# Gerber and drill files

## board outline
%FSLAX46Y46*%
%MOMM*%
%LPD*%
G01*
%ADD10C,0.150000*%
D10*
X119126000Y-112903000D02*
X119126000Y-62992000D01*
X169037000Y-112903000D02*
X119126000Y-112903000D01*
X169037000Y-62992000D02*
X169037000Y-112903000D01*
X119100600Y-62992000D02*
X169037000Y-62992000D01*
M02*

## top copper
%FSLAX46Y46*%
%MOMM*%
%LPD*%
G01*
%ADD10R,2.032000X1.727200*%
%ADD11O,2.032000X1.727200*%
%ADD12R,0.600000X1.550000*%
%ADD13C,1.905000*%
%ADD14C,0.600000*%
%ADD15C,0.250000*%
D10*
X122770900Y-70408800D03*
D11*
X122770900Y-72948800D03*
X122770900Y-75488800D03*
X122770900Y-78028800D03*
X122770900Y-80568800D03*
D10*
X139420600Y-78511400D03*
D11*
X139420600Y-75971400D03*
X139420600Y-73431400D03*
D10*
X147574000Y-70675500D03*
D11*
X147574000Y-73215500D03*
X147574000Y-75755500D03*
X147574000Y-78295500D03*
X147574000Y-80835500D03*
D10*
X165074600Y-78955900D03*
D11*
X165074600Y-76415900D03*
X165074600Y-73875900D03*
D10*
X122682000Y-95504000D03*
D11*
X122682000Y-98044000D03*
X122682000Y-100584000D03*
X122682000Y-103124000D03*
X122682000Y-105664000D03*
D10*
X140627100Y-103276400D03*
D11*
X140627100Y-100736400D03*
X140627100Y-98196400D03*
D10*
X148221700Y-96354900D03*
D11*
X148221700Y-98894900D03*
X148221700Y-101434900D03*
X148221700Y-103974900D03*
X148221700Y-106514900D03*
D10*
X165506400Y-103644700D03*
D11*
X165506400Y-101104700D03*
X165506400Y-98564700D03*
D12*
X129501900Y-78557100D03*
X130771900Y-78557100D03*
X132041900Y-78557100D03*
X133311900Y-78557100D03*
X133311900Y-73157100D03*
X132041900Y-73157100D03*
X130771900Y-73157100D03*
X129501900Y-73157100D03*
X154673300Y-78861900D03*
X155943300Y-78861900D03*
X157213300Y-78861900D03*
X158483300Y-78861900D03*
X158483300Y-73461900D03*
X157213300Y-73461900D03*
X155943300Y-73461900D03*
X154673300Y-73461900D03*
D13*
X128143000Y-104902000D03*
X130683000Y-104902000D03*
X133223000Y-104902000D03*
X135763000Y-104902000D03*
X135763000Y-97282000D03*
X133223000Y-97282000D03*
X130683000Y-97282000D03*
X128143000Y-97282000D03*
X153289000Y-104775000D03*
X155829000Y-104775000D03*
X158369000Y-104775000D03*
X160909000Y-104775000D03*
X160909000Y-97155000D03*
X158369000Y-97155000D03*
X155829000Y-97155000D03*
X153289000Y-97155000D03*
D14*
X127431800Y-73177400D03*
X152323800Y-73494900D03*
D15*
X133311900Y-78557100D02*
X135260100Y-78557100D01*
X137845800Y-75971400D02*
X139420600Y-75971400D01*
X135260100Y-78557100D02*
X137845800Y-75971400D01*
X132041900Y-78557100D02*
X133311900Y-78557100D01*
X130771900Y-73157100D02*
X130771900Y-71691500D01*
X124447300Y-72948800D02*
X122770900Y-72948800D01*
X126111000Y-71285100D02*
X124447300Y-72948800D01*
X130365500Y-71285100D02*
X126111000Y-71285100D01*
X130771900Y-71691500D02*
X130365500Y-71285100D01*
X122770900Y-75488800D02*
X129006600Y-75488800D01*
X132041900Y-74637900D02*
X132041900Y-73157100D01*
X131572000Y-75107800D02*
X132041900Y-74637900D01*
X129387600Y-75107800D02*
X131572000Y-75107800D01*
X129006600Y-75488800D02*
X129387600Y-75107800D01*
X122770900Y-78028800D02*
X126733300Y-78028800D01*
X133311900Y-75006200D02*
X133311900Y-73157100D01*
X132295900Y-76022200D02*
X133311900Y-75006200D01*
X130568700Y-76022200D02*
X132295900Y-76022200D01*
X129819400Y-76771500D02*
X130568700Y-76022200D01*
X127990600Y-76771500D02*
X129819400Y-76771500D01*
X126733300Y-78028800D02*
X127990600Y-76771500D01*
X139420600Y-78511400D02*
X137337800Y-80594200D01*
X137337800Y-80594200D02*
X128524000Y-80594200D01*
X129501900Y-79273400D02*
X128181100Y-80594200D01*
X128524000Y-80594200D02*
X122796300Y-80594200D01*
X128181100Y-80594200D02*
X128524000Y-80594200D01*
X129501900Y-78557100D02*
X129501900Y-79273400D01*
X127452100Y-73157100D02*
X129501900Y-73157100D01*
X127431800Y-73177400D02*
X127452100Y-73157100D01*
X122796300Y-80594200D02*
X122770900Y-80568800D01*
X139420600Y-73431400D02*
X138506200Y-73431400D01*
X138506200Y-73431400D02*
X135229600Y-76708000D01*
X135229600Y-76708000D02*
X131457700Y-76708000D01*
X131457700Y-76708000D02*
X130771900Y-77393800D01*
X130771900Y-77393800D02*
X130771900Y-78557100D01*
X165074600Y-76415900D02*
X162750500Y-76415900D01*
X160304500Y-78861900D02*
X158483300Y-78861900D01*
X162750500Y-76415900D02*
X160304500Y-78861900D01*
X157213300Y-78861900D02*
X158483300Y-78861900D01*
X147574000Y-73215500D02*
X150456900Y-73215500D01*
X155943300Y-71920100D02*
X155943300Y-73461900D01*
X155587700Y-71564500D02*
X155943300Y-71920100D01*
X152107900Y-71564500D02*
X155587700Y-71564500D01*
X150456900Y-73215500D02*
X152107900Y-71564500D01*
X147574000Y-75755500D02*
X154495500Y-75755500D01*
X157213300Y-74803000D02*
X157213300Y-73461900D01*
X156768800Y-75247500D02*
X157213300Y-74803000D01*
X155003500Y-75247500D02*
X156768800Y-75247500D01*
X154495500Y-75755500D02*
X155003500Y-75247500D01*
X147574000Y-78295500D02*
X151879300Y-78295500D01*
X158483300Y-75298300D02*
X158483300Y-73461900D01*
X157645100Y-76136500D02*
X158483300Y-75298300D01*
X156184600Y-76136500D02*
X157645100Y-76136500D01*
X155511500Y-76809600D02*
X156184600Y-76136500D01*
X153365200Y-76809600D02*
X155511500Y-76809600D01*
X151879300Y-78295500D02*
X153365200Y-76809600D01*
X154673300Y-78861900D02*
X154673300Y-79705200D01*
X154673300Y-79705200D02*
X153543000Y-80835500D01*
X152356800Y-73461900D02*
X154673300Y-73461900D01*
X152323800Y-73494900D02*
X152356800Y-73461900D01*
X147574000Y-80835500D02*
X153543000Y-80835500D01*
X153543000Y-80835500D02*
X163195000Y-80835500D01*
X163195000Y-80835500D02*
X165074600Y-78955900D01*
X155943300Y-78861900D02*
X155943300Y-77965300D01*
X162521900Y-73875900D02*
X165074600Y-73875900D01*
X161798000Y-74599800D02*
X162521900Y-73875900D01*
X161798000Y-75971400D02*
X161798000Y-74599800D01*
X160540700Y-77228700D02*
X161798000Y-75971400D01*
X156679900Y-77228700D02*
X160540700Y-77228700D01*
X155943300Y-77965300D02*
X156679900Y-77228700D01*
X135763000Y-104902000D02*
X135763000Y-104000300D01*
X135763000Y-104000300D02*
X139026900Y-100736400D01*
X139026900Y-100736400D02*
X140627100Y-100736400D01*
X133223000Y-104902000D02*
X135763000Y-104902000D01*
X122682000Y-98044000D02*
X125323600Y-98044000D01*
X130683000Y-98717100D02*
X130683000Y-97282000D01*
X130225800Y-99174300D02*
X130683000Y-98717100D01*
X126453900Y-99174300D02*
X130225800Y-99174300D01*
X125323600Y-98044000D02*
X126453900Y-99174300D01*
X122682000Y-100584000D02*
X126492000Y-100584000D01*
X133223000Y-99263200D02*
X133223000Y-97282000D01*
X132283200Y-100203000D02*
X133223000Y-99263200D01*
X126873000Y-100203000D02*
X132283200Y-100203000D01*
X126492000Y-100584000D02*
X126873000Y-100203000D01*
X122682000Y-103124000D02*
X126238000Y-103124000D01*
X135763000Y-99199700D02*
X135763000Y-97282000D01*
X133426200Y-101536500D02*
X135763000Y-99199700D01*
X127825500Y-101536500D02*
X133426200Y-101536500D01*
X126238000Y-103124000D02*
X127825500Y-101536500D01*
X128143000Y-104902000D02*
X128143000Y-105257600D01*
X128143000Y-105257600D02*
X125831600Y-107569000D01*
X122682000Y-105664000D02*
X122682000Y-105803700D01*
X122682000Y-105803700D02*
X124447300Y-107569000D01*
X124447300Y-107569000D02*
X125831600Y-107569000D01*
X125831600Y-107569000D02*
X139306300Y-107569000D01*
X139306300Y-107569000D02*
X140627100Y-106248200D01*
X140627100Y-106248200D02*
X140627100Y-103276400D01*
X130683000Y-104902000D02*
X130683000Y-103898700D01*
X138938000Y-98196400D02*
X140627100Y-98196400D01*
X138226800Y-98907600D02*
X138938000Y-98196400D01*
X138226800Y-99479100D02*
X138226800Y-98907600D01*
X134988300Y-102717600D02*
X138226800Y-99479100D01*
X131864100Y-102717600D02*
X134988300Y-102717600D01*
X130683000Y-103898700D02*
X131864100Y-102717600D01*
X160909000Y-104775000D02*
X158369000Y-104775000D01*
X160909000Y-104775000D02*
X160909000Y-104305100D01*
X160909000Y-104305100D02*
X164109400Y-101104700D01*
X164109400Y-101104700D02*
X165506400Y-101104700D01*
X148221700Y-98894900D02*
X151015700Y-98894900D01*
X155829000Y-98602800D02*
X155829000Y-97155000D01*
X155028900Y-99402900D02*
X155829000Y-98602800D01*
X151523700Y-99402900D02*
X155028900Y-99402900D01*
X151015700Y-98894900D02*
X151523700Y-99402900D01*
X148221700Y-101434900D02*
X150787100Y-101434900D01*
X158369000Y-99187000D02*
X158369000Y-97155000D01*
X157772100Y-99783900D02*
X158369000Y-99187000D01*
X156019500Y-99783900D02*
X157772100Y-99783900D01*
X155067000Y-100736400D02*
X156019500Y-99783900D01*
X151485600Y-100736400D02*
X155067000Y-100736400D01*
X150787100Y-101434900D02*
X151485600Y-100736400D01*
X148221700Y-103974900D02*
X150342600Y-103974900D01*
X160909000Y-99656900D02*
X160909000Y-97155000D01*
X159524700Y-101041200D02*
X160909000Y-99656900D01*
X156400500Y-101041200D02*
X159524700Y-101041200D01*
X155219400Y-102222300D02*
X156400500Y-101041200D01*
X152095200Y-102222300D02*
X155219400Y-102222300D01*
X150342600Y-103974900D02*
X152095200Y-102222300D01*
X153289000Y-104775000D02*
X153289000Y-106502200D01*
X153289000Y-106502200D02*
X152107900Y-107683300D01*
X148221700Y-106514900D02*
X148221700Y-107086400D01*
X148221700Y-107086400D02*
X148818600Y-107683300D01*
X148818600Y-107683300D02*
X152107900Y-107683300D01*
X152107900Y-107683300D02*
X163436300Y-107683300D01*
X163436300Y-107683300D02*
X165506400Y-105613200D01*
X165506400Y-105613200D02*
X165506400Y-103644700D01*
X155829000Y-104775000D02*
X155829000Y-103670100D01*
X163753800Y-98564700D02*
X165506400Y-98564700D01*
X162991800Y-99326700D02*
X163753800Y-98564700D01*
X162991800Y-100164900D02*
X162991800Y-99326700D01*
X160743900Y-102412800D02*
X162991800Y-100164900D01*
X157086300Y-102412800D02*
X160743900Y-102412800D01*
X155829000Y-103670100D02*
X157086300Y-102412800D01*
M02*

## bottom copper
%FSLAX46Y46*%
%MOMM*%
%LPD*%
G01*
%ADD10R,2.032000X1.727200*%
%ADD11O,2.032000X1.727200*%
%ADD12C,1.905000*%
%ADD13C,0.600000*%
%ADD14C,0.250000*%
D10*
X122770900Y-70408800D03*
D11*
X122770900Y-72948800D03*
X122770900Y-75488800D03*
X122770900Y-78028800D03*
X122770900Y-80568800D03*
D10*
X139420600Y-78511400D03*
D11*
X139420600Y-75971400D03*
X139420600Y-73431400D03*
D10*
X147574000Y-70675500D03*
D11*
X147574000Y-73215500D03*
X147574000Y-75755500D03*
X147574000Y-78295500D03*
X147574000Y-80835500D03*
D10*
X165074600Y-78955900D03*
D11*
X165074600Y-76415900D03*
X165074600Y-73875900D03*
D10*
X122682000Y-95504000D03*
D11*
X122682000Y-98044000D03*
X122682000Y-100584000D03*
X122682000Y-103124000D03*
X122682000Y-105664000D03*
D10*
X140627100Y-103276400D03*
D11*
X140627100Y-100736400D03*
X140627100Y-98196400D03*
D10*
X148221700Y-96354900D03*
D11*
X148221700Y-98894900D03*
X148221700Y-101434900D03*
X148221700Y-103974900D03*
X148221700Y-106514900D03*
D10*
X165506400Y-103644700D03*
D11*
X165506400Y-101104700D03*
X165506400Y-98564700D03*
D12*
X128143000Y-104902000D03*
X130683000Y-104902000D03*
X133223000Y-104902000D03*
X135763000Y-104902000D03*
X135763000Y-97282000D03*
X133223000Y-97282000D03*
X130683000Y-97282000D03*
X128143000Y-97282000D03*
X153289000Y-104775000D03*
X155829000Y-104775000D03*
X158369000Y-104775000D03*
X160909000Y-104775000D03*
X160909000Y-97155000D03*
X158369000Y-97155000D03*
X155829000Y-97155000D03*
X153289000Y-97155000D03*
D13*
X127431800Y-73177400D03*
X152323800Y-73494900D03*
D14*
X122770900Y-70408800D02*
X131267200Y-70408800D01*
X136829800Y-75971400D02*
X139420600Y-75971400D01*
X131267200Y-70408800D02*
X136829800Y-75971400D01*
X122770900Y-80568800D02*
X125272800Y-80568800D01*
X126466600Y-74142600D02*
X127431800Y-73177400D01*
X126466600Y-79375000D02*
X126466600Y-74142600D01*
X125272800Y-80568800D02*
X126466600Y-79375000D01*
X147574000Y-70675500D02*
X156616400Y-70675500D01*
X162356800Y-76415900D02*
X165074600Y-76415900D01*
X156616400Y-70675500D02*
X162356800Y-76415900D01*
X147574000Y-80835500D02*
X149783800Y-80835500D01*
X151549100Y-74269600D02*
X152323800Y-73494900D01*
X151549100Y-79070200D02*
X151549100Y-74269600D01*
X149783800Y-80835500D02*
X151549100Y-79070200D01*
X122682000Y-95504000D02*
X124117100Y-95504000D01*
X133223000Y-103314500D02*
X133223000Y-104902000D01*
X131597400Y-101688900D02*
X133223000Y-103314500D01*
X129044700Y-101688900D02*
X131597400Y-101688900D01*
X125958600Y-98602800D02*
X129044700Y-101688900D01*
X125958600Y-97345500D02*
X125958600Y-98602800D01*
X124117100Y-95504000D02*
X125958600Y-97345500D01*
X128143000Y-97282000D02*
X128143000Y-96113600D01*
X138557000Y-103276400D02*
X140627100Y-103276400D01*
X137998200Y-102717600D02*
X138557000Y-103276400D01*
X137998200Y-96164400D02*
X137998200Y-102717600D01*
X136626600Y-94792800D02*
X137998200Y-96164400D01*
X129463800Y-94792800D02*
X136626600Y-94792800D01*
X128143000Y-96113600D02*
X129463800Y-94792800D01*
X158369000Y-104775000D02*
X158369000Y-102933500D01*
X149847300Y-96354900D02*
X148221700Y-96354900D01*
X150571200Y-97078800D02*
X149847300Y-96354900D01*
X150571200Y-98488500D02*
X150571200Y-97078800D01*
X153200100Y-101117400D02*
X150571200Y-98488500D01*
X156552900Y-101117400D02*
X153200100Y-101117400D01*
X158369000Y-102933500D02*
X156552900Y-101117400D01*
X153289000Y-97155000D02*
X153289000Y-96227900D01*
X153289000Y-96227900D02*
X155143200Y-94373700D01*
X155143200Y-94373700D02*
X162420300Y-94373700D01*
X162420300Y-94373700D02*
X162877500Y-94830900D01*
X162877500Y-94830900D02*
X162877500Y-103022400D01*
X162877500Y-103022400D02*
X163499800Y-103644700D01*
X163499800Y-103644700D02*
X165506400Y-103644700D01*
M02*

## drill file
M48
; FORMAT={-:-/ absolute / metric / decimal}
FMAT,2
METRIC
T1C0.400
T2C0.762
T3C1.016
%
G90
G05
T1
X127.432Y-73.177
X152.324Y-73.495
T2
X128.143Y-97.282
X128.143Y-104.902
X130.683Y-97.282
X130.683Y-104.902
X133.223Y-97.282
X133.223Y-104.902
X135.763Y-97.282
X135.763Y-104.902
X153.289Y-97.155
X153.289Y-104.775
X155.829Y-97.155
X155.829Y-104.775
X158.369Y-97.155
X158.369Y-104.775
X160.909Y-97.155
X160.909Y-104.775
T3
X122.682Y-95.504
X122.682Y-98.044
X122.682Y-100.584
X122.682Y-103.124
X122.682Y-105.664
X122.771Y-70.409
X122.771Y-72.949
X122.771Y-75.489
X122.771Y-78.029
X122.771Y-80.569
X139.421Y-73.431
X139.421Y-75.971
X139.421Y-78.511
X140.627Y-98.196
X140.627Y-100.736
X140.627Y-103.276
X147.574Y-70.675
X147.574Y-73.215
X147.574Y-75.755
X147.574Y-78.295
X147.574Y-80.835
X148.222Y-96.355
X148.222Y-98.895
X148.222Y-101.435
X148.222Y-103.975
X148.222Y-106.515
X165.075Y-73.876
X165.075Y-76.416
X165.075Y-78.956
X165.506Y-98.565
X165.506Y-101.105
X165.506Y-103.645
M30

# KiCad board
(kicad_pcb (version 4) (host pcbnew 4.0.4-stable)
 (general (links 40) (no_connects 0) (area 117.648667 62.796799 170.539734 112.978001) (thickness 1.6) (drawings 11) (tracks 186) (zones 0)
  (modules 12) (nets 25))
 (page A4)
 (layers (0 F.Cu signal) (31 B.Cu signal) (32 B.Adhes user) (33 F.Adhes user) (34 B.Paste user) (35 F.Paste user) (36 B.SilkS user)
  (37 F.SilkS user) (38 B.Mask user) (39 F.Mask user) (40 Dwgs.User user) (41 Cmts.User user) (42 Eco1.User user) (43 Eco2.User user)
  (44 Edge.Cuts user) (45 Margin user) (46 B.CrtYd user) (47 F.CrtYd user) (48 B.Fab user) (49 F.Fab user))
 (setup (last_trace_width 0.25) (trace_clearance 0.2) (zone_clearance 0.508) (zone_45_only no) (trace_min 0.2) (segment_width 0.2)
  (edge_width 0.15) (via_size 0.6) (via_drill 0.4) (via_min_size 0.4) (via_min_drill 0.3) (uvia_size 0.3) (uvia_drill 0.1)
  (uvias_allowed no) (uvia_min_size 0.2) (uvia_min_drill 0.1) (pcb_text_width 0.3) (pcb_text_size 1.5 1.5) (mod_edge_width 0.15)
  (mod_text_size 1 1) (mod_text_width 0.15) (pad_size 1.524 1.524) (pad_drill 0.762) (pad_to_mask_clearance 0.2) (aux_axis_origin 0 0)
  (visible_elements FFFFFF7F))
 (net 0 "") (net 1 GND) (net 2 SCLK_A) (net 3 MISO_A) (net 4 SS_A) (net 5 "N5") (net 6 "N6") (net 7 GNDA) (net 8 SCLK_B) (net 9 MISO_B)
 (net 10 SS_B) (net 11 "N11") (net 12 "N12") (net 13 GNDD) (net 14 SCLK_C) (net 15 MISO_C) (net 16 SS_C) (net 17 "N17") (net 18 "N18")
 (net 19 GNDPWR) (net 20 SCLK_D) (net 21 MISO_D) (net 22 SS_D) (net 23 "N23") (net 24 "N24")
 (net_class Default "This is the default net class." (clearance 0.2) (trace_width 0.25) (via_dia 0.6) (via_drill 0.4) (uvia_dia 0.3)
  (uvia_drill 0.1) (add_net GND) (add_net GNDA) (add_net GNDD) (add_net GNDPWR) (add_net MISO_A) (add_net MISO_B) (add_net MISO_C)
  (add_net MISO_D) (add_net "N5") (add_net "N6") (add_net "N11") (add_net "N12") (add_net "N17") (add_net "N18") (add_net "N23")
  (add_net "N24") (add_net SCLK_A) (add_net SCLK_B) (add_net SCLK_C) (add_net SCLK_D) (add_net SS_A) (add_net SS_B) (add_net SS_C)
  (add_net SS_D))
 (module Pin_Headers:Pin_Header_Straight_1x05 (layer F.Cu) (at 122.7709 70.4088)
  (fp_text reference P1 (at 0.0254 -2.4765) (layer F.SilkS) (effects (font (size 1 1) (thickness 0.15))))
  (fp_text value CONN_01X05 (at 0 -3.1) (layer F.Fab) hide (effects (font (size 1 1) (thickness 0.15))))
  (pad 1 thru_hole rect (at 0 0) (size 2.032 1.7272) (drill 1.016) (layers *.Cu *.Mask) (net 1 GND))
  (pad 2 thru_hole oval (at 0 2.54) (size 2.032 1.7272) (drill 1.016) (layers *.Cu *.Mask) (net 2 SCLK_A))
  (pad 3 thru_hole oval (at 0 5.08) (size 2.032 1.7272) (drill 1.016) (layers *.Cu *.Mask) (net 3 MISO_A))
  (pad 4 thru_hole oval (at 0 7.62) (size 2.032 1.7272) (drill 1.016) (layers *.Cu *.Mask) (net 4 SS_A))
  (pad 5 thru_hole oval (at 0 10.16) (size 2.032 1.7272) (drill 1.016) (layers *.Cu *.Mask) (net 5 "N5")))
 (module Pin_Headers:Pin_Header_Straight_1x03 (layer F.Cu) (at 139.4206 78.5114 180)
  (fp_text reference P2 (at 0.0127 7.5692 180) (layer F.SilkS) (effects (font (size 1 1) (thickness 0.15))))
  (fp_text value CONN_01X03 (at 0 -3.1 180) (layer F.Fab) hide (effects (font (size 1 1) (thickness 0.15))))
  (pad 1 thru_hole rect (at 0 0 180) (size 2.032 1.7272) (drill 1.016) (layers *.Cu *.Mask) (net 5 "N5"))
  (pad 2 thru_hole oval (at 0 2.54 180) (size 2.032 1.7272) (drill 1.016) (layers *.Cu *.Mask) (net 1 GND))
  (pad 3 thru_hole oval (at 0 5.08 180) (size 2.032 1.7272) (drill 1.016) (layers *.Cu *.Mask) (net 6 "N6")))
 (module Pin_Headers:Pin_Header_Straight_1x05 (layer F.Cu) (at 147.574 70.6755)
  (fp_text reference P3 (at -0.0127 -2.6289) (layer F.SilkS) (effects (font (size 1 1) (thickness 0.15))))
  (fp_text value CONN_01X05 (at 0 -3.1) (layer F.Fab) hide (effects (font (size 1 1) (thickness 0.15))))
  (pad 1 thru_hole rect (at 0 0) (size 2.032 1.7272) (drill 1.016) (layers *.Cu *.Mask) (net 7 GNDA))
  (pad 2 thru_hole oval (at 0 2.54) (size 2.032 1.7272) (drill 1.016) (layers *.Cu *.Mask) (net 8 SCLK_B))
  (pad 3 thru_hole oval (at 0 5.08) (size 2.032 1.7272) (drill 1.016) (layers *.Cu *.Mask) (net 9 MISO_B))
  (pad 4 thru_hole oval (at 0 7.62) (size 2.032 1.7272) (drill 1.016) (layers *.Cu *.Mask) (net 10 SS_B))
  (pad 5 thru_hole oval (at 0 10.16) (size 2.032 1.7272) (drill 1.016) (layers *.Cu *.Mask) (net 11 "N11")))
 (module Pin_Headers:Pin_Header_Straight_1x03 (layer F.Cu) (at 165.0746 78.9559 180)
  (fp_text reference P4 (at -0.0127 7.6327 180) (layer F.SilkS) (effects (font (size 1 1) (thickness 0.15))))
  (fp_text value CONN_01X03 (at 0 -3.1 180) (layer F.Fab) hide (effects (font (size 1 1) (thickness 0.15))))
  (pad 1 thru_hole rect (at 0 0 180) (size 2.032 1.7272) (drill 1.016) (layers *.Cu *.Mask) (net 11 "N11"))
  (pad 2 thru_hole oval (at 0 2.54 180) (size 2.032 1.7272) (drill 1.016) (layers *.Cu *.Mask) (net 7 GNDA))
  (pad 3 thru_hole oval (at 0 5.08 180) (size 2.032 1.7272) (drill 1.016) (layers *.Cu *.Mask) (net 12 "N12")))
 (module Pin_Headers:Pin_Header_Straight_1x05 (layer F.Cu) (at 122.682 95.504)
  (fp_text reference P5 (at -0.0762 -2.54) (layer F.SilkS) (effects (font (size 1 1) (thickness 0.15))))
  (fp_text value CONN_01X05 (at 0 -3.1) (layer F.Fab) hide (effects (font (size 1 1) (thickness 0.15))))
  (pad 1 thru_hole rect (at 0 0) (size 2.032 1.7272) (drill 1.016) (layers *.Cu *.Mask) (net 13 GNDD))
  (pad 2 thru_hole oval (at 0 2.54) (size 2.032 1.7272) (drill 1.016) (layers *.Cu *.Mask) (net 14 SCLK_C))
  (pad 3 thru_hole oval (at 0 5.08) (size 2.032 1.7272) (drill 1.016) (layers *.Cu *.Mask) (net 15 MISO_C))
  (pad 4 thru_hole oval (at 0 7.62) (size 2.032 1.7272) (drill 1.016) (layers *.Cu *.Mask) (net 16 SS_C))
  (pad 5 thru_hole oval (at 0 10.16) (size 2.032 1.7272) (drill 1.016) (layers *.Cu *.Mask) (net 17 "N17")))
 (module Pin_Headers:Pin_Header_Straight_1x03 (layer F.Cu) (at 140.6271 103.2764 180)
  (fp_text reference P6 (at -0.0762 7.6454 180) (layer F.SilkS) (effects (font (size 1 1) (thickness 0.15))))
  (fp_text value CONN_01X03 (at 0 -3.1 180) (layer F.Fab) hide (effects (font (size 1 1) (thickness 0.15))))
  (pad 1 thru_hole rect (at 0 0 180) (size 2.032 1.7272) (drill 1.016) (layers *.Cu *.Mask) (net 17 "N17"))
  (pad 2 thru_hole oval (at 0 2.54 180) (size 2.032 1.7272) (drill 1.016) (layers *.Cu *.Mask) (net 13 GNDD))
  (pad 3 thru_hole oval (at 0 5.08 180) (size 2.032 1.7272) (drill 1.016) (layers *.Cu *.Mask) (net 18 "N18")))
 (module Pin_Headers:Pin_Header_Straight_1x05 (layer F.Cu) (at 148.2217 96.3549)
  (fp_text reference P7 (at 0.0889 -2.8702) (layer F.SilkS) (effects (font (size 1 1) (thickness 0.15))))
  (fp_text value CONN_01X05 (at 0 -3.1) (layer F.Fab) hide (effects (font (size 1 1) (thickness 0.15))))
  (pad 1 thru_hole rect (at 0 0) (size 2.032 1.7272) (drill 1.016) (layers *.Cu *.Mask) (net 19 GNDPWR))
  (pad 2 thru_hole oval (at 0 2.54) (size 2.032 1.7272) (drill 1.016) (layers *.Cu *.Mask) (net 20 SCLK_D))
  (pad 3 thru_hole oval (at 0 5.08) (size 2.032 1.7272) (drill 1.016) (layers *.Cu *.Mask) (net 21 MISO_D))
  (pad 4 thru_hole oval (at 0 7.62) (size 2.032 1.7272) (drill 1.016) (layers *.Cu *.Mask) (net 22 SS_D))
  (pad 5 thru_hole oval (at 0 10.16) (size 2.032 1.7272) (drill 1.016) (layers *.Cu *.Mask) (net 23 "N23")))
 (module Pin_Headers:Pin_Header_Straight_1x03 (layer F.Cu) (at 165.5064 103.6447 180)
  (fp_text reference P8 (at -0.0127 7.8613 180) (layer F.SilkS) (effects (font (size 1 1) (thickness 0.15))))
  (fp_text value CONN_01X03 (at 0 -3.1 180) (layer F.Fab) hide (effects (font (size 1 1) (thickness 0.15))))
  (pad 1 thru_hole rect (at 0 0 180) (size 2.032 1.7272) (drill 1.016) (layers *.Cu *.Mask) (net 23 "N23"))
  (pad 2 thru_hole oval (at 0 2.54 180) (size 2.032 1.7272) (drill 1.016) (layers *.Cu *.Mask) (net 19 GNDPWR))
  (pad 3 thru_hole oval (at 0 5.08 180) (size 2.032 1.7272) (drill 1.016) (layers *.Cu *.Mask) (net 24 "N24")))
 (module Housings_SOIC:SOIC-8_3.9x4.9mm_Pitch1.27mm (layer F.Cu) (at 131.4069 75.8571 90)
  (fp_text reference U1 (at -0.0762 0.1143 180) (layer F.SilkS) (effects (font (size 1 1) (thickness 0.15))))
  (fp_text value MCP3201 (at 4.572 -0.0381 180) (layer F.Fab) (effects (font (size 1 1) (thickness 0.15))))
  (pad 1 smd rect (at -2.7 -1.905 90) (size 1.55 0.6) (layers F.Cu F.Paste F.Mask) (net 5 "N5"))
  (pad 2 smd rect (at -2.7 -0.635 90) (size 1.55 0.6) (layers F.Cu F.Paste F.Mask) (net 6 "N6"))
  (pad 3 smd rect (at -2.7 0.635 90) (size 1.55 0.6) (layers F.Cu F.Paste F.Mask) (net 1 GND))
  (pad 4 smd rect (at -2.7 1.905 90) (size 1.55 0.6) (layers F.Cu F.Paste F.Mask) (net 1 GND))
  (pad 5 smd rect (at 2.7 1.905 90) (size 1.55 0.6) (layers F.Cu F.Paste F.Mask) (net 4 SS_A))
  (pad 6 smd rect (at 2.7 0.635 90) (size 1.55 0.6) (layers F.Cu F.Paste F.Mask) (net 3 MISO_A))
  (pad 7 smd rect (at 2.7 -0.635 90) (size 1.55 0.6) (layers F.Cu F.Paste F.Mask) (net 2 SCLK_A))
  (pad 8 smd rect (at 2.7 -1.905 90) (size 1.55 0.6) (layers F.Cu F.Paste F.Mask) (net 5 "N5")))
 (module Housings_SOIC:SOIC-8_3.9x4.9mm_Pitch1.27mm (layer F.Cu) (at 156.5783 76.1619 90)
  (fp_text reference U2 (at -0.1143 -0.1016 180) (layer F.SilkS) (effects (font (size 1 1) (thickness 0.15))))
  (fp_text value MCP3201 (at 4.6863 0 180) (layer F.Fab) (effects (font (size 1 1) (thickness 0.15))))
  (pad 1 smd rect (at -2.7 -1.905 90) (size 1.55 0.6) (layers F.Cu F.Paste F.Mask) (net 11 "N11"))
  (pad 2 smd rect (at -2.7 -0.635 90) (size 1.55 0.6) (layers F.Cu F.Paste F.Mask) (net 12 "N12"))
  (pad 3 smd rect (at -2.7 0.635 90) (size 1.55 0.6) (layers F.Cu F.Paste F.Mask) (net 7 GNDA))
  (pad 4 smd rect (at -2.7 1.905 90) (size 1.55 0.6) (layers F.Cu F.Paste F.Mask) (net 7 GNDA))
  (pad 5 smd rect (at 2.7 1.905 90) (size 1.55 0.6) (layers F.Cu F.Paste F.Mask) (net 10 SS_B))
  (pad 6 smd rect (at 2.7 0.635 90) (size 1.55 0.6) (layers F.Cu F.Paste F.Mask) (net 9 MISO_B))
  (pad 7 smd rect (at 2.7 -0.635 90) (size 1.55 0.6) (layers F.Cu F.Paste F.Mask) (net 8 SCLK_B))
  (pad 8 smd rect (at 2.7 -1.905 90) (size 1.55 0.6) (layers F.Cu F.Paste F.Mask) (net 11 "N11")))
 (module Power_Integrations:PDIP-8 (layer F.Cu) (at 131.953 101.092)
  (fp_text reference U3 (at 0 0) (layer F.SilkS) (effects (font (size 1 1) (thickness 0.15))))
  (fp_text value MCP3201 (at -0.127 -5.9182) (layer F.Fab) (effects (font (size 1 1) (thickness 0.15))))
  (pad 1 thru_hole circle (at -3.81 3.81) (size 1.905 1.905) (drill 0.762) (layers *.Cu *.Mask) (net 17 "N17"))
  (pad 2 thru_hole circle (at -1.27 3.81) (size 1.905 1.905) (drill 0.762) (layers *.Cu *.Mask) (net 18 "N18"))
  (pad 3 thru_hole circle (at 1.27 3.81) (size 1.905 1.905) (drill 0.762) (layers *.Cu *.Mask) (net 13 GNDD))
  (pad 4 thru_hole circle (at 3.81 3.81) (size 1.905 1.905) (drill 0.762) (layers *.Cu *.Mask) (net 13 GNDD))
  (pad 5 thru_hole circle (at 3.81 -3.81) (size 1.905 1.905) (drill 0.762) (layers *.Cu *.Mask) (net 16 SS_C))
  (pad 6 thru_hole circle (at 1.27 -3.81) (size 1.905 1.905) (drill 0.762) (layers *.Cu *.Mask) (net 15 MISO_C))
  (pad 7 thru_hole circle (at -1.27 -3.81) (size 1.905 1.905) (drill 0.762) (layers *.Cu *.Mask) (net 14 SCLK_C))
  (pad 8 thru_hole circle (at -3.81 -3.81) (size 1.905 1.905) (drill 0.762) (layers *.Cu *.Mask) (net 17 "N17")))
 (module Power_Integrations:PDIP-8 (layer F.Cu) (at 157.099 100.965)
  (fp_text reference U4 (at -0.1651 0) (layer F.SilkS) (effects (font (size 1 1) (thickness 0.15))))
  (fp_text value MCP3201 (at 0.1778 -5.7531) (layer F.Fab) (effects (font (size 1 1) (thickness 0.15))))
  (pad 1 thru_hole circle (at -3.81 3.81) (size 1.905 1.905) (drill 0.762) (layers *.Cu *.Mask) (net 23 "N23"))
  (pad 2 thru_hole circle (at -1.27 3.81) (size 1.905 1.905) (drill 0.762) (layers *.Cu *.Mask) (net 24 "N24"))
  (pad 3 thru_hole circle (at 1.27 3.81) (size 1.905 1.905) (drill 0.762) (layers *.Cu *.Mask) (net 19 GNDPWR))
  (pad 4 thru_hole circle (at 3.81 3.81) (size 1.905 1.905) (drill 0.762) (layers *.Cu *.Mask) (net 19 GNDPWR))
  (pad 5 thru_hole circle (at 3.81 -3.81) (size 1.905 1.905) (drill 0.762) (layers *.Cu *.Mask) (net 22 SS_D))
  (pad 6 thru_hole circle (at 1.27 -3.81) (size 1.905 1.905) (drill 0.762) (layers *.Cu *.Mask) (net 21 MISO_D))
  (pad 7 thru_hole circle (at -1.27 -3.81) (size 1.905 1.905) (drill 0.762) (layers *.Cu *.Mask) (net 20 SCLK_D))
  (pad 8 thru_hole circle (at -3.81 -3.81) (size 1.905 1.905) (drill 0.762) (layers *.Cu *.Mask) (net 23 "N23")))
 (gr_line (start 119.126 112.903) (end 119.126 62.992) (angle 90) (layer Edge.Cuts) (width 0.15))
 (gr_line (start 169.037 112.903) (end 119.126 112.903) (angle 90) (layer Edge.Cuts) (width 0.15))
 (gr_line (start 169.037 62.992) (end 169.037 112.903) (angle 90) (layer Edge.Cuts) (width 0.15))
 (gr_line (start 119.1006 62.992) (end 169.037 62.992) (angle 90) (layer Edge.Cuts) (width 0.15))
 (segment (start 122.7709 70.4088) (end 131.2672 70.4088) (width 0.25) (layer B.Cu) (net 1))
 (segment (start 136.8298 75.9714) (end 139.4206 75.9714) (width 0.25) (layer B.Cu) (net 1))
 (segment (start 131.2672 70.4088) (end 136.8298 75.9714) (width 0.25) (layer B.Cu) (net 1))
 (segment (start 133.3119 78.5571) (end 135.2601 78.5571) (width 0.25) (layer F.Cu) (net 1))
 (segment (start 137.8458 75.9714) (end 139.4206 75.9714) (width 0.25) (layer F.Cu) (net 1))
 (segment (start 135.2601 78.5571) (end 137.8458 75.9714) (width 0.25) (layer F.Cu) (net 1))
 (segment (start 132.0419 78.5571) (end 133.3119 78.5571) (width 0.25) (layer F.Cu) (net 1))
 (segment (start 130.7719 73.1571) (end 130.7719 71.6915) (width 0.25) (layer F.Cu) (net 2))
 (segment (start 124.4473 72.9488) (end 122.7709 72.9488) (width 0.25) (layer F.Cu) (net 2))
 (segment (start 126.111 71.2851) (end 124.4473 72.9488) (width 0.25) (layer F.Cu) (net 2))
 (segment (start 130.3655 71.2851) (end 126.111 71.2851) (width 0.25) (layer F.Cu) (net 2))
 (segment (start 130.7719 71.6915) (end 130.3655 71.2851) (width 0.25) (layer F.Cu) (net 2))
 (segment (start 122.7709 75.4888) (end 129.0066 75.4888) (width 0.25) (layer F.Cu) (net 3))
 (segment (start 132.0419 74.6379) (end 132.0419 73.1571) (width 0.25) (layer F.Cu) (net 3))
 (segment (start 131.572 75.1078) (end 132.0419 74.6379) (width 0.25) (layer F.Cu) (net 3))
 (segment (start 129.3876 75.1078) (end 131.572 75.1078) (width 0.25) (layer F.Cu) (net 3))
 (segment (start 129.0066 75.4888) (end 129.3876 75.1078) (width 0.25) (layer F.Cu) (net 3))
 (segment (start 122.7709 78.0288) (end 126.7333 78.0288) (width 0.25) (layer F.Cu) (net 4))
 (segment (start 133.3119 75.0062) (end 133.3119 73.1571) (width 0.25) (layer F.Cu) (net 4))
 (segment (start 132.2959 76.0222) (end 133.3119 75.0062) (width 0.25) (layer F.Cu) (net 4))
 (segment (start 130.5687 76.0222) (end 132.2959 76.0222) (width 0.25) (layer F.Cu) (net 4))
 (segment (start 129.8194 76.7715) (end 130.5687 76.0222) (width 0.25) (layer F.Cu) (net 4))
 (segment (start 127.9906 76.7715) (end 129.8194 76.7715) (width 0.25) (layer F.Cu) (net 4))
 (segment (start 126.7333 78.0288) (end 127.9906 76.7715) (width 0.25) (layer F.Cu) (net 4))
 (segment (start 139.4206 78.5114) (end 137.3378 80.5942) (width 0.25) (layer F.Cu) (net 5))
 (segment (start 137.3378 80.5942) (end 128.524 80.5942) (width 0.25) (layer F.Cu) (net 5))
 (segment (start 129.5019 79.2734) (end 128.1811 80.5942) (width 0.25) (layer F.Cu) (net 5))
 (segment (start 128.524 80.5942) (end 122.7963 80.5942) (width 0.25) (layer F.Cu) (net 5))
 (segment (start 128.1811 80.5942) (end 128.524 80.5942) (width 0.25) (layer F.Cu) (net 5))
 (segment (start 129.5019 78.5571) (end 129.5019 79.2734) (width 0.25) (layer F.Cu) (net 5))
 (segment (start 122.7709 80.5688) (end 125.2728 80.5688) (width 0.25) (layer B.Cu) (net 5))
 (segment (start 127.4521 73.1571) (end 129.5019 73.1571) (width 0.25) (layer F.Cu) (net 5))
 (segment (start 127.4318 73.1774) (end 127.4521 73.1571) (width 0.25) (layer F.Cu) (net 5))
 (via (at 127.4318 73.1774) (size 0.6) (drill 0.4) (layers F.Cu B.Cu) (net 5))
 (segment (start 126.4666 74.1426) (end 127.4318 73.1774) (width 0.25) (layer B.Cu) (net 5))
 (segment (start 126.4666 79.375) (end 126.4666 74.1426) (width 0.25) (layer B.Cu) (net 5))
 (segment (start 125.2728 80.5688) (end 126.4666 79.375) (width 0.25) (layer B.Cu) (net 5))
 (segment (start 122.7963 80.5942) (end 122.7709 80.5688) (width 0.25) (layer F.Cu) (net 5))
 (segment (start 139.4206 73.4314) (end 138.5062 73.4314) (width 0.25) (layer F.Cu) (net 6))
 (segment (start 138.5062 73.4314) (end 135.2296 76.708) (width 0.25) (layer F.Cu) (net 6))
 (segment (start 135.2296 76.708) (end 131.4577 76.708) (width 0.25) (layer F.Cu) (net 6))
 (segment (start 131.4577 76.708) (end 130.7719 77.3938) (width 0.25) (layer F.Cu) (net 6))
 (segment (start 130.7719 77.3938) (end 130.7719 78.5571) (width 0.25) (layer F.Cu) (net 6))
 (segment (start 165.0746 76.4159) (end 162.7505 76.4159) (width 0.25) (layer F.Cu) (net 7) (status 400000))
 (segment (start 160.3045 78.8619) (end 158.4833 78.8619) (width 0.25) (layer F.Cu) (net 7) (status 800000))
 (segment (start 162.7505 76.4159) (end 160.3045 78.8619) (width 0.25) (layer F.Cu) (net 7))
 (segment (start 157.2133 78.8619) (end 158.4833 78.8619) (width 0.25) (layer F.Cu) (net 7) (status C00000))
 (segment (start 147.574 70.6755) (end 156.6164 70.6755) (width 0.25) (layer B.Cu) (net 7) (status 400000))
 (segment (start 162.3568 76.4159) (end 165.0746 76.4159) (width 0.25) (layer B.Cu) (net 7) (status 800000))
 (segment (start 156.6164 70.6755) (end 162.3568 76.4159) (width 0.25) (layer B.Cu) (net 7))
 (segment (start 147.574 73.2155) (end 150.4569 73.2155) (width 0.25) (layer F.Cu) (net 8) (status 400000))
 (segment (start 155.9433 71.9201) (end 155.9433 73.4619) (width 0.25) (layer F.Cu) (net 8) (status 800000))
 (segment (start 155.5877 71.5645) (end 155.9433 71.9201) (width 0.25) (layer F.Cu) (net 8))
 (segment (start 152.1079 71.5645) (end 155.5877 71.5645) (width 0.25) (layer F.Cu) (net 8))
 (segment (start 150.4569 73.2155) (end 152.1079 71.5645) (width 0.25) (layer F.Cu) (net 8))
 (segment (start 147.574 75.7555) (end 154.4955 75.7555) (width 0.25) (layer F.Cu) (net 9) (status 400000))
 (segment (start 157.2133 74.803) (end 157.2133 73.4619) (width 0.25) (layer F.Cu) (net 9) (status 800000))
 (segment (start 156.7688 75.2475) (end 157.2133 74.803) (width 0.25) (layer F.Cu) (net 9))
 (segment (start 155.0035 75.2475) (end 156.7688 75.2475) (width 0.25) (layer F.Cu) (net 9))
 (segment (start 154.4955 75.7555) (end 155.0035 75.2475) (width 0.25) (layer F.Cu) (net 9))
 (segment (start 147.574 78.2955) (end 151.8793 78.2955) (width 0.25) (layer F.Cu) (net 10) (status 400000))
 (segment (start 158.4833 75.2983) (end 158.4833 73.4619) (width 0.25) (layer F.Cu) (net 10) (status 800000))
 (segment (start 157.6451 76.1365) (end 158.4833 75.2983) (width 0.25) (layer F.Cu) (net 10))
 (segment (start 156.1846 76.1365) (end 157.6451 76.1365) (width 0.25) (layer F.Cu) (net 10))
 (segment (start 155.5115 76.8096) (end 156.1846 76.1365) (width 0.25) (layer F.Cu) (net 10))
 (segment (start 153.3652 76.8096) (end 155.5115 76.8096) (width 0.25) (layer F.Cu) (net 10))
 (segment (start 151.8793 78.2955) (end 153.3652 76.8096) (width 0.25) (layer F.Cu) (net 10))
 (segment (start 154.6733 78.8619) (end 154.6733 79.7052) (width 0.25) (layer F.Cu) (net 11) (status 400000))
 (segment (start 154.6733 79.7052) (end 153.543 80.8355) (width 0.25) (layer F.Cu) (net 11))
 (segment (start 147.574 80.8355) (end 149.7838 80.8355) (width 0.25) (layer B.Cu) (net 11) (status 400000))
 (segment (start 152.3568 73.4619) (end 154.6733 73.4619) (width 0.25) (layer F.Cu) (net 11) (status 800000))
 (segment (start 152.3238 73.4949) (end 152.3568 73.4619) (width 0.25) (layer F.Cu) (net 11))
 (via (at 152.3238 73.4949) (size 0.6) (drill 0.4) (layers F.Cu B.Cu) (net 11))
 (segment (start 151.5491 74.2696) (end 152.3238 73.4949) (width 0.25) (layer B.Cu) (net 11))
 (segment (start 151.5491 79.0702) (end 151.5491 74.2696) (width 0.25) (layer B.Cu) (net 11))
 (segment (start 149.7838 80.8355) (end 151.5491 79.0702) (width 0.25) (layer B.Cu) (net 11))
 (segment (start 147.574 80.8355) (end 153.543 80.8355) (width 0.25) (layer F.Cu) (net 11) (status 400000))
 (segment (start 153.543 80.8355) (end 163.195 80.8355) (width 0.25) (layer F.Cu) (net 11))
 (segment (start 163.195 80.8355) (end 165.0746 78.9559) (width 0.25) (layer F.Cu) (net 11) (status 800000))
 (segment (start 155.9433 78.8619) (end 155.9433 77.9653) (width 0.25) (layer F.Cu) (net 12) (status 400000))
 (segment (start 162.5219 73.8759) (end 165.0746 73.8759) (width 0.25) (layer F.Cu) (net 12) (status 800000))
 (segment (start 161.798 74.5998) (end 162.5219 73.8759) (width 0.25) (layer F.Cu) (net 12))
 (segment (start 161.798 75.9714) (end 161.798 74.5998) (width 0.25) (layer F.Cu) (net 12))
 (segment (start 160.5407 77.2287) (end 161.798 75.9714) (width 0.25) (layer F.Cu) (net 12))
 (segment (start 156.6799 77.2287) (end 160.5407 77.2287) (width 0.25) (layer F.Cu) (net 12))
 (segment (start 155.9433 77.9653) (end 156.6799 77.2287) (width 0.25) (layer F.Cu) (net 12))
 (segment (start 122.682 95.504) (end 124.1171 95.504) (width 0.25) (layer B.Cu) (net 13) (status 400000))
 (segment (start 133.223 103.3145) (end 133.223 104.902) (width 0.25) (layer B.Cu) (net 13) (status 800000))
 (segment (start 131.5974 101.6889) (end 133.223 103.3145) (width 0.25) (layer B.Cu) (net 13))
 (segment (start 129.0447 101.6889) (end 131.5974 101.6889) (width 0.25) (layer B.Cu) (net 13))
 (segment (start 125.9586 98.6028) (end 129.0447 101.6889) (width 0.25) (layer B.Cu) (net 13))
 (segment (start 125.9586 97.3455) (end 125.9586 98.6028) (width 0.25) (layer B.Cu) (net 13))
 (segment (start 124.1171 95.504) (end 125.9586 97.3455) (width 0.25) (layer B.Cu) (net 13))
 (segment (start 135.763 104.902) (end 135.763 104.0003) (width 0.25) (layer F.Cu) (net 13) (status C00000))
 (segment (start 135.763 104.0003) (end 139.0269 100.7364) (width 0.25) (layer F.Cu) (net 13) (status 400000))
 (segment (start 139.0269 100.7364) (end 140.6271 100.7364) (width 0.25) (layer F.Cu) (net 13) (status 800000))
 (segment (start 133.223 104.902) (end 135.763 104.902) (width 0.25) (layer F.Cu) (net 13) (status C00000))
 (segment (start 122.682 98.044) (end 125.3236 98.044) (width 0.25) (layer F.Cu) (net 14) (status 400000))
 (segment (start 130.683 98.7171) (end 130.683 97.282) (width 0.25) (layer F.Cu) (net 14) (status 800000))
 (segment (start 130.2258 99.1743) (end 130.683 98.7171) (width 0.25) (layer F.Cu) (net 14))
 (segment (start 126.4539 99.1743) (end 130.2258 99.1743) (width 0.25) (layer F.Cu) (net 14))
 (segment (start 125.3236 98.044) (end 126.4539 99.1743) (width 0.25) (layer F.Cu) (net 14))
 (segment (start 122.682 100.584) (end 126.492 100.584) (width 0.25) (layer F.Cu) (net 15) (status 400000))
 (segment (start 133.223 99.2632) (end 133.223 97.282) (width 0.25) (layer F.Cu) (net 15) (status 800000))
 (segment (start 132.2832 100.203) (end 133.223 99.2632) (width 0.25) (layer F.Cu) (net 15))
 (segment (start 126.873 100.203) (end 132.2832 100.203) (width 0.25) (layer F.Cu) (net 15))
 (segment (start 126.492 100.584) (end 126.873 100.203) (width 0.25) (layer F.Cu) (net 15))
 (segment (start 122.682 103.124) (end 126.238 103.124) (width 0.25) (layer F.Cu) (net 16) (status 400000))
 (segment (start 135.763 99.1997) (end 135.763 97.282) (width 0.25) (layer F.Cu) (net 16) (status 800000))
 (segment (start 133.4262 101.5365) (end 135.763 99.1997) (width 0.25) (layer F.Cu) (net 16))
 (segment (start 127.8255 101.5365) (end 133.4262 101.5365) (width 0.25) (layer F.Cu) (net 16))
 (segment (start 126.238 103.124) (end 127.8255 101.5365) (width 0.25) (layer F.Cu) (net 16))
 (segment (start 128.143 97.282) (end 128.143 96.1136) (width 0.25) (layer B.Cu) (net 17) (status 400000))
 (segment (start 138.557 103.2764) (end 140.6271 103.2764) (width 0.25) (layer B.Cu) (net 17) (status 800000))
 (segment (start 137.9982 102.7176) (end 138.557 103.2764) (width 0.25) (layer B.Cu) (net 17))
 (segment (start 137.9982 96.1644) (end 137.9982 102.7176) (width 0.25) (layer B.Cu) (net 17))
 (segment (start 136.6266 94.7928) (end 137.9982 96.1644) (width 0.25) (layer B.Cu) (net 17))
 (segment (start 129.4638 94.7928) (end 136.6266 94.7928) (width 0.25) (layer B.Cu) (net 17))
 (segment (start 128.143 96.1136) (end 129.4638 94.7928) (width 0.25) (layer B.Cu) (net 17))
 (segment (start 128.143 104.902) (end 128.143 105.2576) (width 0.25) (layer F.Cu) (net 17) (status C00000))
 (segment (start 128.143 105.2576) (end 125.8316 107.569) (width 0.25) (layer F.Cu) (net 17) (status 400000))
 (segment (start 122.682 105.664) (end 122.682 105.8037) (width 0.25) (layer F.Cu) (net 17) (status C00000))
 (segment (start 122.682 105.8037) (end 124.4473 107.569) (width 0.25) (layer F.Cu) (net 17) (status 400000))
 (segment (start 124.4473 107.569) (end 125.8316 107.569) (width 0.25) (layer F.Cu) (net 17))
 (segment (start 125.8316 107.569) (end 139.3063 107.569) (width 0.25) (layer F.Cu) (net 17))
 (segment (start 139.3063 107.569) (end 140.6271 106.2482) (width 0.25) (layer F.Cu) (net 17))
 (segment (start 140.6271 106.2482) (end 140.6271 103.2764) (width 0.25) (layer F.Cu) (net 17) (status 800000))
 (segment (start 130.683 104.902) (end 130.683 103.8987) (width 0.25) (layer F.Cu) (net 18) (status 400000))
 (segment (start 138.938 98.1964) (end 140.6271 98.1964) (width 0.25) (layer F.Cu) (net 18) (status 800000))
 (segment (start 138.2268 98.9076) (end 138.938 98.1964) (width 0.25) (layer F.Cu) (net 18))
 (segment (start 138.2268 99.4791) (end 138.2268 98.9076) (width 0.25) (layer F.Cu) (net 18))
 (segment (start 134.9883 102.7176) (end 138.2268 99.4791) (width 0.25) (layer F.Cu) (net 18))
 (segment (start 131.8641 102.7176) (end 134.9883 102.7176) (width 0.25) (layer F.Cu) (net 18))
 (segment (start 130.683 103.8987) (end 131.8641 102.7176) (width 0.25) (layer F.Cu) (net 18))
 (segment (start 158.369 104.775) (end 158.369 102.9335) (width 0.25) (layer B.Cu) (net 19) (status 400000))
 (segment (start 149.8473 96.3549) (end 148.2217 96.3549) (width 0.25) (layer B.Cu) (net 19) (status 800000))
 (segment (start 150.5712 97.0788) (end 149.8473 96.3549) (width 0.25) (layer B.Cu) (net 19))
 (segment (start 150.5712 98.4885) (end 150.5712 97.0788) (width 0.25) (layer B.Cu) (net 19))
 (segment (start 153.2001 101.1174) (end 150.5712 98.4885) (width 0.25) (layer B.Cu) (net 19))
 (segment (start 156.5529 101.1174) (end 153.2001 101.1174) (width 0.25) (layer B.Cu) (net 19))
 (segment (start 158.369 102.9335) (end 156.5529 101.1174) (width 0.25) (layer B.Cu) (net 19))
 (segment (start 160.909 104.775) (end 158.369 104.775) (width 0.25) (layer F.Cu) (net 19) (status C00000))
 (segment (start 160.909 104.775) (end 160.909 104.3051) (width 0.25) (layer F.Cu) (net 19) (status C00000))
 (segment (start 160.909 104.3051) (end 164.1094 101.1047) (width 0.25) (layer F.Cu) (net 19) (status 400000))
 (segment (start 164.1094 101.1047) (end 165.5064 101.1047) (width 0.25) (layer F.Cu) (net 19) (status 800000))
 (segment (start 148.2217 98.8949) (end 151.0157 98.8949) (width 0.25) (layer F.Cu) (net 20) (status 400000))
 (segment (start 155.829 98.6028) (end 155.829 97.155) (width 0.25) (layer F.Cu) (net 20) (status 800000))
 (segment (start 155.0289 99.4029) (end 155.829 98.6028) (width 0.25) (layer F.Cu) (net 20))
 (segment (start 151.5237 99.4029) (end 155.0289 99.4029) (width 0.25) (layer F.Cu) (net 20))
 (segment (start 151.0157 98.8949) (end 151.5237 99.4029) (width 0.25) (layer F.Cu) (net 20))
 (segment (start 148.2217 101.4349) (end 150.7871 101.4349) (width 0.25) (layer F.Cu) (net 21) (status 400000))
 (segment (start 158.369 99.187) (end 158.369 97.155) (width 0.25) (layer F.Cu) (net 21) (status 800000))
 (segment (start 157.7721 99.7839) (end 158.369 99.187) (width 0.25) (layer F.Cu) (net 21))
 (segment (start 156.0195 99.7839) (end 157.7721 99.7839) (width 0.25) (layer F.Cu) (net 21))
 (segment (start 155.067 100.7364) (end 156.0195 99.7839) (width 0.25) (layer F.Cu) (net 21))
 (segment (start 151.4856 100.7364) (end 155.067 100.7364) (width 0.25) (layer F.Cu) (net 21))
 (segment (start 150.7871 101.4349) (end 151.4856 100.7364) (width 0.25) (layer F.Cu) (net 21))
 (segment (start 148.2217 103.9749) (end 150.3426 103.9749) (width 0.25) (layer F.Cu) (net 22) (status 400000))
 (segment (start 160.909 99.6569) (end 160.909 97.155) (width 0.25) (layer F.Cu) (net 22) (status 800000))
 (segment (start 159.5247 101.0412) (end 160.909 99.6569) (width 0.25) (layer F.Cu) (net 22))
 (segment (start 156.4005 101.0412) (end 159.5247 101.0412) (width 0.25) (layer F.Cu) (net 22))
 (segment (start 155.2194 102.2223) (end 156.4005 101.0412) (width 0.25) (layer F.Cu) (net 22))
 (segment (start 152.0952 102.2223) (end 155.2194 102.2223) (width 0.25) (layer F.Cu) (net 22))
 (segment (start 150.3426 103.9749) (end 152.0952 102.2223) (width 0.25) (layer F.Cu) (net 22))
 (segment (start 153.289 97.155) (end 153.289 96.2279) (width 0.25) (layer B.Cu) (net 23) (status C00000))
 (segment (start 153.289 96.2279) (end 155.1432 94.3737) (width 0.25) (layer B.Cu) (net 23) (status 400000))
 (segment (start 155.1432 94.3737) (end 162.4203 94.3737) (width 0.25) (layer B.Cu) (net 23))
 (segment (start 162.4203 94.3737) (end 162.8775 94.8309) (width 0.25) (layer B.Cu) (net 23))
 (segment (start 162.8775 94.8309) (end 162.8775 103.0224) (width 0.25) (layer B.Cu) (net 23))
 (segment (start 162.8775 103.0224) (end 163.4998 103.6447) (width 0.25) (layer B.Cu) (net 23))
 (segment (start 163.4998 103.6447) (end 165.5064 103.6447) (width 0.25) (layer B.Cu) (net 23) (status 800000))
 (segment (start 153.289 104.775) (end 153.289 106.5022) (width 0.25) (layer F.Cu) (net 23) (status 400000))
 (segment (start 153.289 106.5022) (end 152.1079 107.6833) (width 0.25) (layer F.Cu) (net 23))
 (segment (start 148.2217 106.5149) (end 148.2217 107.0864) (width 0.25) (layer F.Cu) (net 23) (status C00000))
 (segment (start 148.2217 107.0864) (end 148.8186 107.6833) (width 0.25) (layer F.Cu) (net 23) (status 400000))
 (segment (start 148.8186 107.6833) (end 152.1079 107.6833) (width 0.25) (layer F.Cu) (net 23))
 (segment (start 152.1079 107.6833) (end 163.4363 107.6833) (width 0.25) (layer F.Cu) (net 23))
 (segment (start 163.4363 107.6833) (end 165.5064 105.6132) (width 0.25) (layer F.Cu) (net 23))
 (segment (start 165.5064 105.6132) (end 165.5064 103.6447) (width 0.25) (layer F.Cu) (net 23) (status 800000))
 (segment (start 155.829 104.775) (end 155.829 103.6701) (width 0.25) (layer F.Cu) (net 24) (status 400000))
 (segment (start 163.7538 98.5647) (end 165.5064 98.5647) (width 0.25) (layer F.Cu) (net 24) (status 800000))
 (segment (start 162.9918 99.3267) (end 163.7538 98.5647) (width 0.25) (layer F.Cu) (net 24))
 (segment (start 162.9918 100.1649) (end 162.9918 99.3267) (width 0.25) (layer F.Cu) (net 24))
 (segment (start 160.7439 102.4128) (end 162.9918 100.1649) (width 0.25) (layer F.Cu) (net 24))
 (segment (start 157.0863 102.4128) (end 160.7439 102.4128) (width 0.25) (layer F.Cu) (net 24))
 (segment (start 155.829 103.6701) (end 157.0863 102.4128) (width 0.25) (layer F.Cu) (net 24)))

